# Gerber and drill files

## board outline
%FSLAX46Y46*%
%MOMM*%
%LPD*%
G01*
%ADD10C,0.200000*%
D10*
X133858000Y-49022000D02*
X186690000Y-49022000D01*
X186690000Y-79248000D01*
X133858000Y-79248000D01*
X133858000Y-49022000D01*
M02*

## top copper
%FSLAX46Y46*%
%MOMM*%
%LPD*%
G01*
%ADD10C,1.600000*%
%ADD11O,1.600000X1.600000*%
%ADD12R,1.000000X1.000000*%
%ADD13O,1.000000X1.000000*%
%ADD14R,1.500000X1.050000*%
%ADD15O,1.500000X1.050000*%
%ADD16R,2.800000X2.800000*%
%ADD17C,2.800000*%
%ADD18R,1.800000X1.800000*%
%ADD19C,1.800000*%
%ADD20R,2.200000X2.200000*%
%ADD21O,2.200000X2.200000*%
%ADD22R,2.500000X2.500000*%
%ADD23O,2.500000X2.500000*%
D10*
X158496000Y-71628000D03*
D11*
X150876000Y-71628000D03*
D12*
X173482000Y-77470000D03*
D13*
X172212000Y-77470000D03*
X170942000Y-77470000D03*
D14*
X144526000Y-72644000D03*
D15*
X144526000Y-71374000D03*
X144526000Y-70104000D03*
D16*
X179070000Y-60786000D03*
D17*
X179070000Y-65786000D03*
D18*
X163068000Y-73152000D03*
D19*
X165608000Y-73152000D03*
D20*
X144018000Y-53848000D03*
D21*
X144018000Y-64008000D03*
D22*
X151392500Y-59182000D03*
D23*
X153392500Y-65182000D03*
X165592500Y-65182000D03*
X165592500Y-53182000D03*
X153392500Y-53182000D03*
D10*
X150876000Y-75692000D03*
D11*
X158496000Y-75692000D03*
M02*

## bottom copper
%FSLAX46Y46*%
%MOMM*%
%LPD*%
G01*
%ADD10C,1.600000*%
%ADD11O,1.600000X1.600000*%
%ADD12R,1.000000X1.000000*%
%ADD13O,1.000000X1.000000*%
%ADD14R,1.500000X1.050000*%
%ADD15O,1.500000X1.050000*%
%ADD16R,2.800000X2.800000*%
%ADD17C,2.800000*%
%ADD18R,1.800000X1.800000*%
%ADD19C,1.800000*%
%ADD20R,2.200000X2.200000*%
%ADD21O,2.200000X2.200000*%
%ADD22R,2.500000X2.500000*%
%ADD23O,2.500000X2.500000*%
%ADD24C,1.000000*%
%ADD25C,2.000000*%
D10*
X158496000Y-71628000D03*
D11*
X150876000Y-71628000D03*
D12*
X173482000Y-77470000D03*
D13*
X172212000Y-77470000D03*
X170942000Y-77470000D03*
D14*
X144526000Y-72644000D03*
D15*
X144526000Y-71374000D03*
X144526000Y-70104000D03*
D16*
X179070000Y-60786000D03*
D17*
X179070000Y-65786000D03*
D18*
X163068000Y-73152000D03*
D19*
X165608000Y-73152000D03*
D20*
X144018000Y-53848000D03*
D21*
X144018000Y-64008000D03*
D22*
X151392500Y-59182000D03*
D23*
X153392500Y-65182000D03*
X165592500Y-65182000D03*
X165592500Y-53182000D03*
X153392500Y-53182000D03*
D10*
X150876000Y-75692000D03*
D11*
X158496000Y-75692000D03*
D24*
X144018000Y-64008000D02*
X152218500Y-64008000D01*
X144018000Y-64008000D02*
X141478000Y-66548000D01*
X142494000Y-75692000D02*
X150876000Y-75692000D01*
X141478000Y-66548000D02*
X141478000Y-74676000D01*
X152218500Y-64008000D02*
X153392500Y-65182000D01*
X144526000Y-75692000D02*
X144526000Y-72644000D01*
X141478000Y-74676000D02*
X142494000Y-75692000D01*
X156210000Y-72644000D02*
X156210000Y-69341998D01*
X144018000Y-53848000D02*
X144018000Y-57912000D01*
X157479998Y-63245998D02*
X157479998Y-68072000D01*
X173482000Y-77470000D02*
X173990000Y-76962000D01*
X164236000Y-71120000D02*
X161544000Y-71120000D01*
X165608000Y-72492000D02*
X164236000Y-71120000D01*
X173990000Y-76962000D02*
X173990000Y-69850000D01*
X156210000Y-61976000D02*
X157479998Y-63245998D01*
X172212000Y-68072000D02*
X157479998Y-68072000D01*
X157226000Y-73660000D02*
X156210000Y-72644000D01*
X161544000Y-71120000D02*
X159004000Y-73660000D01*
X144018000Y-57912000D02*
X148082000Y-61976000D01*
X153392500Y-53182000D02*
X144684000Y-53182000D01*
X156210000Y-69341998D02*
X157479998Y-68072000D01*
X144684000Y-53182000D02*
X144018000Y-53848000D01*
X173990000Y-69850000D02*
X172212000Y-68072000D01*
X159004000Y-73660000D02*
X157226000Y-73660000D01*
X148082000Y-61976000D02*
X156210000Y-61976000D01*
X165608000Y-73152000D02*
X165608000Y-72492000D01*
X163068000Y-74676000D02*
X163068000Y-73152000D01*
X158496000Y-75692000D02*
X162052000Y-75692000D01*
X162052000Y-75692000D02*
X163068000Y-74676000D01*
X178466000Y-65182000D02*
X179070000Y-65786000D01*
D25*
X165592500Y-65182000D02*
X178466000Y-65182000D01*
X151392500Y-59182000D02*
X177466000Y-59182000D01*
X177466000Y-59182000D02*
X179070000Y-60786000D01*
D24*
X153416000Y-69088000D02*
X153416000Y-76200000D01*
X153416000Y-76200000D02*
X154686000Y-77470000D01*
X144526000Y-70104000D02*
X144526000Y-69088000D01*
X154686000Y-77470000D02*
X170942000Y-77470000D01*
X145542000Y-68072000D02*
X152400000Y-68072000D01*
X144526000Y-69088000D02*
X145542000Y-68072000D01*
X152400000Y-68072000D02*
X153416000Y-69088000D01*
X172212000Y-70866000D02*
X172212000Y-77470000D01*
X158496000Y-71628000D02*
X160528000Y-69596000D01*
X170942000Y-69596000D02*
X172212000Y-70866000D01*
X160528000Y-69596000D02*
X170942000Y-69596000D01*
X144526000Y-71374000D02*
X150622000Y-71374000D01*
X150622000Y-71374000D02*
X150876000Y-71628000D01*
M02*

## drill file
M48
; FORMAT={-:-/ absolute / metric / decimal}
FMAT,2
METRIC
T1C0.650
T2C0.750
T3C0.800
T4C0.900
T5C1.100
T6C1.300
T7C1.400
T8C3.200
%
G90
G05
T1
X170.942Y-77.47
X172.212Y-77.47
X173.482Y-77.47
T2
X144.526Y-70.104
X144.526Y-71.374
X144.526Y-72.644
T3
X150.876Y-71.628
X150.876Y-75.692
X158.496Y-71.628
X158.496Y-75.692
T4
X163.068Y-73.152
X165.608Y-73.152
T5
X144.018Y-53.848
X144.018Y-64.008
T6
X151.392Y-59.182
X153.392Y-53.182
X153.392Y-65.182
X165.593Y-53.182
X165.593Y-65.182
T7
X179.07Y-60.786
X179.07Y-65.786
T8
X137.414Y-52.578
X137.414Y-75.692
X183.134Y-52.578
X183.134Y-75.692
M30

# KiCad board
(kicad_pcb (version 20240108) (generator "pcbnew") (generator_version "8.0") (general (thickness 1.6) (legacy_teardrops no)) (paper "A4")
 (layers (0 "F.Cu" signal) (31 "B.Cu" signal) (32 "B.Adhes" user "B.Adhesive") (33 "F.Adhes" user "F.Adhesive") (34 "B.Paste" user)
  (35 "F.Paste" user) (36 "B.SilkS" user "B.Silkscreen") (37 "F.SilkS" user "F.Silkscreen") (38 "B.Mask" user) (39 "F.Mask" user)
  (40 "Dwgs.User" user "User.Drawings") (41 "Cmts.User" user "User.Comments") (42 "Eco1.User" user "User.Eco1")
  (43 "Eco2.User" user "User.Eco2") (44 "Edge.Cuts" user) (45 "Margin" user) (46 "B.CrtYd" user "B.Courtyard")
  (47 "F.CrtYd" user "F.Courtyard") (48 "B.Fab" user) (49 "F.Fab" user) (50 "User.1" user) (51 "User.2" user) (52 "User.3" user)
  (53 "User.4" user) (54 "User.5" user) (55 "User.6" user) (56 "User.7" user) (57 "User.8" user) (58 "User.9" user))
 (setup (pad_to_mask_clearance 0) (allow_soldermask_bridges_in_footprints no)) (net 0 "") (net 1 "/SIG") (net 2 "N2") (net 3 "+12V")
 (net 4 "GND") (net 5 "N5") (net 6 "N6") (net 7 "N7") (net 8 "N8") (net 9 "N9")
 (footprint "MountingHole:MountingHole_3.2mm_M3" (layer "F.Cu") (at 183.134 75.692)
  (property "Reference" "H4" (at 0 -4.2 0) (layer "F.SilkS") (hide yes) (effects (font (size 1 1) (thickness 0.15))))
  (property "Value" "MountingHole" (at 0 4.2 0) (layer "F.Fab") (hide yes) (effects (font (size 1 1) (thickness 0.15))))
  (pad "" np_thru_hole circle (at 0 0) (size 3.2 3.2) (drill 3.2) (layers "*.Cu" "*.Mask")))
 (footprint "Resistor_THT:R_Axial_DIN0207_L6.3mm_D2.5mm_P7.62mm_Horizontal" (layer "F.Cu") (at 158.496 71.628 180)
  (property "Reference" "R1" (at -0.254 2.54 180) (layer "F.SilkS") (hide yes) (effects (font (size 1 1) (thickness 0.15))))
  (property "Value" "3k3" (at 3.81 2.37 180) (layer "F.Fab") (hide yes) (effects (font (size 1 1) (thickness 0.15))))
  (pad "1" thru_hole circle (at 0 0 180) (size 1.6 1.6) (drill 0.8) (layers "*.Cu" "*.Mask") (remove_unused_layers no) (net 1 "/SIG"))
  (pad "2" thru_hole oval (at 7.62 0 180) (size 1.6 1.6) (drill 0.8) (layers "*.Cu" "*.Mask") (remove_unused_layers no) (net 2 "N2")))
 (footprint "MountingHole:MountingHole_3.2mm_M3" (layer "F.Cu") (at 137.414 52.578)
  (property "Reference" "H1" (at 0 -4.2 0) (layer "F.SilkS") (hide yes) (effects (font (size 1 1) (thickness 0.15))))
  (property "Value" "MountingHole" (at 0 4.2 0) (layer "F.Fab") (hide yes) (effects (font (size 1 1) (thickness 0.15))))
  (pad "" np_thru_hole circle (at 0 0) (size 3.2 3.2) (drill 3.2) (layers "*.Cu" "*.Mask")))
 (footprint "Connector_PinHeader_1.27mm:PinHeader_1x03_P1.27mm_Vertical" (layer "F.Cu") (at 173.482 77.47 -90)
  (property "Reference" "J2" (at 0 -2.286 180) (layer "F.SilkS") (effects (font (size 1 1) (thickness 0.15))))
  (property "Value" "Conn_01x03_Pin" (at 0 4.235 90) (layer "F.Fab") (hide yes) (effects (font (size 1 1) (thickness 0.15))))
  (pad "1" thru_hole rect (at 0 0 270) (size 1 1) (drill 0.65) (layers "*.Cu" "*.Mask") (remove_unused_layers no) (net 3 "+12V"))
  (pad "2" thru_hole oval (at 0 1.27 270) (size 1 1) (drill 0.65) (layers "*.Cu" "*.Mask") (remove_unused_layers no) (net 1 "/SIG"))
  (pad "3" thru_hole oval (at 0 2.54 270) (size 1 1) (drill 0.65) (layers "*.Cu" "*.Mask") (remove_unused_layers no) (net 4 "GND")))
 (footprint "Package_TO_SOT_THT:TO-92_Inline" (layer "F.Cu") (at 144.526 72.644 90)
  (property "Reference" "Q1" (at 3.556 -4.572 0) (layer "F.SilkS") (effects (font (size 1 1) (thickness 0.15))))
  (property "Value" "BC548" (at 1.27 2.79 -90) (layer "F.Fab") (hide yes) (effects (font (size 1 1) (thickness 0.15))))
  (pad "1" thru_hole rect (at 0 0 90) (size 1.05 1.5) (drill 0.75) (layers "*.Cu" "*.Mask") (remove_unused_layers no) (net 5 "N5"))
  (pad "2" thru_hole oval (at 1.27 0 90) (size 1.05 1.5) (drill 0.75) (layers "*.Cu" "*.Mask") (remove_unused_layers no) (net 2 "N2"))
  (pad "3" thru_hole oval (at 2.54 0 90) (size 1.05 1.5) (drill 0.75) (layers "*.Cu" "*.Mask") (remove_unused_layers no) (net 4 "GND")))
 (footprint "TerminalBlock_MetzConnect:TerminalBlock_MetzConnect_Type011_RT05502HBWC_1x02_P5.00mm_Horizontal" (layer "F.Cu")
  (at 179.07 60.786 -90)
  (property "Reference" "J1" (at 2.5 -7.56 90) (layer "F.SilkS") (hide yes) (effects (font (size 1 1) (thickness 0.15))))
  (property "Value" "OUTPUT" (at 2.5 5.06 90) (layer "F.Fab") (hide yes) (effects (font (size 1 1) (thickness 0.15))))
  (pad "1" thru_hole rect (at 0 0 270) (size 2.8 2.8) (drill 1.4) (layers "*.Cu" "*.Mask") (remove_unused_layers no) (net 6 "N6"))
  (pad "2" thru_hole circle (at 5 0 270) (size 2.8 2.8) (drill 1.4) (layers "*.Cu" "*.Mask") (remove_unused_layers no) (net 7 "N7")))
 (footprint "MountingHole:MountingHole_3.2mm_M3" (layer "F.Cu") (at 137.414 75.692)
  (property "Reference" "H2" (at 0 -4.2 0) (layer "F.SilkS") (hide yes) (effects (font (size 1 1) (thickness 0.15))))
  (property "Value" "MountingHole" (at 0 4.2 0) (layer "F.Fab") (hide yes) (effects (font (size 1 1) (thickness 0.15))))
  (pad "" np_thru_hole circle (at 0 0) (size 3.2 3.2) (drill 3.2) (layers "*.Cu" "*.Mask")))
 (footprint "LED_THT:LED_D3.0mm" (layer "F.Cu") (at 163.068 73.152)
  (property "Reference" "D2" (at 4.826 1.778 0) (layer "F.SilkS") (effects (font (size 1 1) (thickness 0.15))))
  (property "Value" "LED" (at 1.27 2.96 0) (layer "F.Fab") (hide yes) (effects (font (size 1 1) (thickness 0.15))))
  (pad "1" thru_hole rect (at 0 0) (size 1.8 1.8) (drill 0.9) (layers "*.Cu" "*.Mask") (remove_unused_layers no) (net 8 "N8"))
  (pad "2" thru_hole circle (at 2.54 0) (size 1.8 1.8) (drill 0.9) (layers "*.Cu" "*.Mask") (remove_unused_layers no) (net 3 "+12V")))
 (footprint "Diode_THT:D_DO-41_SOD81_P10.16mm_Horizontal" (layer "F.Cu") (at 144.018 53.848 -90)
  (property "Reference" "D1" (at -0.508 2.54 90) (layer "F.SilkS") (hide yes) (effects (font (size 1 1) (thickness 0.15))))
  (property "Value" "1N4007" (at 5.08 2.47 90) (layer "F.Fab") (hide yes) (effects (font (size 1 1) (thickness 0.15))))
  (pad "1" thru_hole rect (at 0 0 270) (size 2.2 2.2) (drill 1.1) (layers "*.Cu" "*.Mask") (remove_unused_layers no) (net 3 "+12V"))
  (pad "2" thru_hole oval (at 10.16 0 270) (size 2.2 2.2) (drill 1.1) (layers "*.Cu" "*.Mask") (remove_unused_layers no) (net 5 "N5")))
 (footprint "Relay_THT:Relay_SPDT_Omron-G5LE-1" (layer "F.Cu") (at 151.3925 59.182 90)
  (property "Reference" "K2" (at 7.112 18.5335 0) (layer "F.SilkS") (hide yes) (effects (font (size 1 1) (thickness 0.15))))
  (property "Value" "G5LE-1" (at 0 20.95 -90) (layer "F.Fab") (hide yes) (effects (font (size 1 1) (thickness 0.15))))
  (pad "1" thru_hole rect (at 0 0 90) (size 2.5 2.5) (drill 1.3) (layers "*.Cu" "*.Mask") (remove_unused_layers no) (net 6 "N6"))
  (pad "2" thru_hole oval (at -6 2 90) (size 2.5 2.5) (drill 1.3) (layers "*.Cu" "*.Mask") (remove_unused_layers no) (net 5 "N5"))
  (pad "3" thru_hole oval (at -6 14.2 90) (size 2.5 2.5) (drill 1.3) (layers "*.Cu" "*.Mask") (remove_unused_layers no) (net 7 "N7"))
  (pad "4" thru_hole oval (at 6 14.2 90) (size 2.5 2.5) (drill 1.3) (layers "*.Cu" "*.Mask") (remove_unused_layers no) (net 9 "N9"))
  (pad "5" thru_hole oval (at 6 2 90) (size 2.5 2.5) (drill 1.3) (layers "*.Cu" "*.Mask") (remove_unused_layers no) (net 3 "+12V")))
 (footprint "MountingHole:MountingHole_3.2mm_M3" (layer "F.Cu") (at 183.134 52.578)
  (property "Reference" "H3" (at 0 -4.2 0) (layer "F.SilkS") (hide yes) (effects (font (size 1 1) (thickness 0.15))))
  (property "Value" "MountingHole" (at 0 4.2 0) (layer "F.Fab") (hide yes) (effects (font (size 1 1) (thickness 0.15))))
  (pad "" np_thru_hole circle (at 0 0) (size 3.2 3.2) (drill 3.2) (layers "*.Cu" "*.Mask")))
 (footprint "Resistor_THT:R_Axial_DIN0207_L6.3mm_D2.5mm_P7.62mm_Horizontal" (layer "F.Cu") (at 150.876 75.692)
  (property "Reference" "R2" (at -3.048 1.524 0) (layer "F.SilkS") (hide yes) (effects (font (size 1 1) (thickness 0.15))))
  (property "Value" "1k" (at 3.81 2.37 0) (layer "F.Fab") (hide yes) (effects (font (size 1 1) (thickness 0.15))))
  (pad "1" thru_hole circle (at 0 0) (size 1.6 1.6) (drill 0.8) (layers "*.Cu" "*.Mask") (remove_unused_layers no) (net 5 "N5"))
  (pad "2" thru_hole oval (at 7.62 0) (size 1.6 1.6) (drill 0.8) (layers "*.Cu" "*.Mask") (remove_unused_layers no) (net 8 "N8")))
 (gr_rect (start 133.858 49.022) (end 186.69 79.248) (stroke (width 0.2) (type default)) (fill none) (layer "Edge.Cuts"))
 (segment (start 144.018 64.008) (end 152.2185 64.008) (width 1) (layer "B.Cu") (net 5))
 (segment (start 144.018 64.008) (end 141.478 66.548) (width 1) (layer "B.Cu") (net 5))
 (segment (start 142.494 75.692) (end 150.876 75.692) (width 1) (layer "B.Cu") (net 5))
 (segment (start 141.478 66.548) (end 141.478 74.676) (width 1) (layer "B.Cu") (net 5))
 (segment (start 152.2185 64.008) (end 153.3925 65.182) (width 1) (layer "B.Cu") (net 5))
 (segment (start 144.526 75.692) (end 144.526 72.644) (width 1) (layer "B.Cu") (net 5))
 (segment (start 141.478 74.676) (end 142.494 75.692) (width 1) (layer "B.Cu") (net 5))
 (segment (start 156.21 72.644) (end 156.21 69.341998) (width 1) (layer "B.Cu") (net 3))
 (segment (start 144.018 53.848) (end 144.018 57.912) (width 1) (layer "B.Cu") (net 3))
 (segment (start 157.479998 63.245998) (end 157.479998 68.072) (width 1) (layer "B.Cu") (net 3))
 (segment (start 173.482 77.47) (end 173.99 76.962) (width 1) (layer "B.Cu") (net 3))
 (segment (start 164.236 71.12) (end 161.544 71.12) (width 1) (layer "B.Cu") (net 3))
 (segment (start 165.608 72.492) (end 164.236 71.12) (width 1) (layer "B.Cu") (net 3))
 (segment (start 173.99 76.962) (end 173.99 69.85) (width 1) (layer "B.Cu") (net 3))
 (segment (start 156.21 61.976) (end 157.479998 63.245998) (width 1) (layer "B.Cu") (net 3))
 (segment (start 172.212 68.072) (end 157.479998 68.072) (width 1) (layer "B.Cu") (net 3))
 (segment (start 157.226 73.66) (end 156.21 72.644) (width 1) (layer "B.Cu") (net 3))
 (segment (start 161.544 71.12) (end 159.004 73.66) (width 1) (layer "B.Cu") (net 3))
 (segment (start 144.018 57.912) (end 148.082 61.976) (width 1) (layer "B.Cu") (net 3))
 (segment (start 153.3925 53.182) (end 144.684 53.182) (width 1) (layer "B.Cu") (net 3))
 (segment (start 156.21 69.341998) (end 157.479998 68.072) (width 1) (layer "B.Cu") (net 3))
 (segment (start 144.684 53.182) (end 144.018 53.848) (width 1) (layer "B.Cu") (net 3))
 (segment (start 173.99 69.85) (end 172.212 68.072) (width 1) (layer "B.Cu") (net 3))
 (segment (start 159.004 73.66) (end 157.226 73.66) (width 1) (layer "B.Cu") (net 3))
 (segment (start 148.082 61.976) (end 156.21 61.976) (width 1) (layer "B.Cu") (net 3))
 (segment (start 165.608 73.152) (end 165.608 72.492) (width 1) (layer "B.Cu") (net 3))
 (segment (start 163.068 74.676) (end 163.068 73.152) (width 1) (layer "B.Cu") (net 8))
 (segment (start 158.496 75.692) (end 162.052 75.692) (width 1) (layer "B.Cu") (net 8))
 (segment (start 162.052 75.692) (end 163.068 74.676) (width 1) (layer "B.Cu") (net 8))
 (segment (start 178.466 65.182) (end 179.07 65.786) (width 1) (layer "B.Cu") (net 7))
 (segment (start 165.5925 65.182) (end 178.466 65.182) (width 2) (layer "B.Cu") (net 7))
 (segment (start 151.3925 59.182) (end 177.466 59.182) (width 2) (layer "B.Cu") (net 6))
 (segment (start 177.466 59.182) (end 179.07 60.786) (width 2) (layer "B.Cu") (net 6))
 (segment (start 153.416 69.088) (end 153.416 76.2) (width 1) (layer "B.Cu") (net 4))
 (segment (start 153.416 76.2) (end 154.686 77.47) (width 1) (layer "B.Cu") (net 4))
 (segment (start 144.526 70.104) (end 144.526 69.088) (width 1) (layer "B.Cu") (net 4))
 (segment (start 154.686 77.47) (end 170.942 77.47) (width 1) (layer "B.Cu") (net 4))
 (segment (start 145.542 68.072) (end 152.4 68.072) (width 1) (layer "B.Cu") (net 4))
 (segment (start 144.526 69.088) (end 145.542 68.072) (width 1) (layer "B.Cu") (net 4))
 (segment (start 152.4 68.072) (end 153.416 69.088) (width 1) (layer "B.Cu") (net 4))
 (segment (start 172.212 70.866) (end 172.212 77.47) (width 1) (layer "B.Cu") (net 1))
 (segment (start 158.496 71.628) (end 160.528 69.596) (width 1) (layer "B.Cu") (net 1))
 (segment (start 170.942 69.596) (end 172.212 70.866) (width 1) (layer "B.Cu") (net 1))
 (segment (start 160.528 69.596) (end 170.942 69.596) (width 1) (layer "B.Cu") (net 1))
 (segment (start 144.526 71.374) (end 150.622 71.374) (width 1) (layer "B.Cu") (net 2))
 (segment (start 150.622 71.374) (end 150.876 71.628) (width 1) (layer "B.Cu") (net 2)))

